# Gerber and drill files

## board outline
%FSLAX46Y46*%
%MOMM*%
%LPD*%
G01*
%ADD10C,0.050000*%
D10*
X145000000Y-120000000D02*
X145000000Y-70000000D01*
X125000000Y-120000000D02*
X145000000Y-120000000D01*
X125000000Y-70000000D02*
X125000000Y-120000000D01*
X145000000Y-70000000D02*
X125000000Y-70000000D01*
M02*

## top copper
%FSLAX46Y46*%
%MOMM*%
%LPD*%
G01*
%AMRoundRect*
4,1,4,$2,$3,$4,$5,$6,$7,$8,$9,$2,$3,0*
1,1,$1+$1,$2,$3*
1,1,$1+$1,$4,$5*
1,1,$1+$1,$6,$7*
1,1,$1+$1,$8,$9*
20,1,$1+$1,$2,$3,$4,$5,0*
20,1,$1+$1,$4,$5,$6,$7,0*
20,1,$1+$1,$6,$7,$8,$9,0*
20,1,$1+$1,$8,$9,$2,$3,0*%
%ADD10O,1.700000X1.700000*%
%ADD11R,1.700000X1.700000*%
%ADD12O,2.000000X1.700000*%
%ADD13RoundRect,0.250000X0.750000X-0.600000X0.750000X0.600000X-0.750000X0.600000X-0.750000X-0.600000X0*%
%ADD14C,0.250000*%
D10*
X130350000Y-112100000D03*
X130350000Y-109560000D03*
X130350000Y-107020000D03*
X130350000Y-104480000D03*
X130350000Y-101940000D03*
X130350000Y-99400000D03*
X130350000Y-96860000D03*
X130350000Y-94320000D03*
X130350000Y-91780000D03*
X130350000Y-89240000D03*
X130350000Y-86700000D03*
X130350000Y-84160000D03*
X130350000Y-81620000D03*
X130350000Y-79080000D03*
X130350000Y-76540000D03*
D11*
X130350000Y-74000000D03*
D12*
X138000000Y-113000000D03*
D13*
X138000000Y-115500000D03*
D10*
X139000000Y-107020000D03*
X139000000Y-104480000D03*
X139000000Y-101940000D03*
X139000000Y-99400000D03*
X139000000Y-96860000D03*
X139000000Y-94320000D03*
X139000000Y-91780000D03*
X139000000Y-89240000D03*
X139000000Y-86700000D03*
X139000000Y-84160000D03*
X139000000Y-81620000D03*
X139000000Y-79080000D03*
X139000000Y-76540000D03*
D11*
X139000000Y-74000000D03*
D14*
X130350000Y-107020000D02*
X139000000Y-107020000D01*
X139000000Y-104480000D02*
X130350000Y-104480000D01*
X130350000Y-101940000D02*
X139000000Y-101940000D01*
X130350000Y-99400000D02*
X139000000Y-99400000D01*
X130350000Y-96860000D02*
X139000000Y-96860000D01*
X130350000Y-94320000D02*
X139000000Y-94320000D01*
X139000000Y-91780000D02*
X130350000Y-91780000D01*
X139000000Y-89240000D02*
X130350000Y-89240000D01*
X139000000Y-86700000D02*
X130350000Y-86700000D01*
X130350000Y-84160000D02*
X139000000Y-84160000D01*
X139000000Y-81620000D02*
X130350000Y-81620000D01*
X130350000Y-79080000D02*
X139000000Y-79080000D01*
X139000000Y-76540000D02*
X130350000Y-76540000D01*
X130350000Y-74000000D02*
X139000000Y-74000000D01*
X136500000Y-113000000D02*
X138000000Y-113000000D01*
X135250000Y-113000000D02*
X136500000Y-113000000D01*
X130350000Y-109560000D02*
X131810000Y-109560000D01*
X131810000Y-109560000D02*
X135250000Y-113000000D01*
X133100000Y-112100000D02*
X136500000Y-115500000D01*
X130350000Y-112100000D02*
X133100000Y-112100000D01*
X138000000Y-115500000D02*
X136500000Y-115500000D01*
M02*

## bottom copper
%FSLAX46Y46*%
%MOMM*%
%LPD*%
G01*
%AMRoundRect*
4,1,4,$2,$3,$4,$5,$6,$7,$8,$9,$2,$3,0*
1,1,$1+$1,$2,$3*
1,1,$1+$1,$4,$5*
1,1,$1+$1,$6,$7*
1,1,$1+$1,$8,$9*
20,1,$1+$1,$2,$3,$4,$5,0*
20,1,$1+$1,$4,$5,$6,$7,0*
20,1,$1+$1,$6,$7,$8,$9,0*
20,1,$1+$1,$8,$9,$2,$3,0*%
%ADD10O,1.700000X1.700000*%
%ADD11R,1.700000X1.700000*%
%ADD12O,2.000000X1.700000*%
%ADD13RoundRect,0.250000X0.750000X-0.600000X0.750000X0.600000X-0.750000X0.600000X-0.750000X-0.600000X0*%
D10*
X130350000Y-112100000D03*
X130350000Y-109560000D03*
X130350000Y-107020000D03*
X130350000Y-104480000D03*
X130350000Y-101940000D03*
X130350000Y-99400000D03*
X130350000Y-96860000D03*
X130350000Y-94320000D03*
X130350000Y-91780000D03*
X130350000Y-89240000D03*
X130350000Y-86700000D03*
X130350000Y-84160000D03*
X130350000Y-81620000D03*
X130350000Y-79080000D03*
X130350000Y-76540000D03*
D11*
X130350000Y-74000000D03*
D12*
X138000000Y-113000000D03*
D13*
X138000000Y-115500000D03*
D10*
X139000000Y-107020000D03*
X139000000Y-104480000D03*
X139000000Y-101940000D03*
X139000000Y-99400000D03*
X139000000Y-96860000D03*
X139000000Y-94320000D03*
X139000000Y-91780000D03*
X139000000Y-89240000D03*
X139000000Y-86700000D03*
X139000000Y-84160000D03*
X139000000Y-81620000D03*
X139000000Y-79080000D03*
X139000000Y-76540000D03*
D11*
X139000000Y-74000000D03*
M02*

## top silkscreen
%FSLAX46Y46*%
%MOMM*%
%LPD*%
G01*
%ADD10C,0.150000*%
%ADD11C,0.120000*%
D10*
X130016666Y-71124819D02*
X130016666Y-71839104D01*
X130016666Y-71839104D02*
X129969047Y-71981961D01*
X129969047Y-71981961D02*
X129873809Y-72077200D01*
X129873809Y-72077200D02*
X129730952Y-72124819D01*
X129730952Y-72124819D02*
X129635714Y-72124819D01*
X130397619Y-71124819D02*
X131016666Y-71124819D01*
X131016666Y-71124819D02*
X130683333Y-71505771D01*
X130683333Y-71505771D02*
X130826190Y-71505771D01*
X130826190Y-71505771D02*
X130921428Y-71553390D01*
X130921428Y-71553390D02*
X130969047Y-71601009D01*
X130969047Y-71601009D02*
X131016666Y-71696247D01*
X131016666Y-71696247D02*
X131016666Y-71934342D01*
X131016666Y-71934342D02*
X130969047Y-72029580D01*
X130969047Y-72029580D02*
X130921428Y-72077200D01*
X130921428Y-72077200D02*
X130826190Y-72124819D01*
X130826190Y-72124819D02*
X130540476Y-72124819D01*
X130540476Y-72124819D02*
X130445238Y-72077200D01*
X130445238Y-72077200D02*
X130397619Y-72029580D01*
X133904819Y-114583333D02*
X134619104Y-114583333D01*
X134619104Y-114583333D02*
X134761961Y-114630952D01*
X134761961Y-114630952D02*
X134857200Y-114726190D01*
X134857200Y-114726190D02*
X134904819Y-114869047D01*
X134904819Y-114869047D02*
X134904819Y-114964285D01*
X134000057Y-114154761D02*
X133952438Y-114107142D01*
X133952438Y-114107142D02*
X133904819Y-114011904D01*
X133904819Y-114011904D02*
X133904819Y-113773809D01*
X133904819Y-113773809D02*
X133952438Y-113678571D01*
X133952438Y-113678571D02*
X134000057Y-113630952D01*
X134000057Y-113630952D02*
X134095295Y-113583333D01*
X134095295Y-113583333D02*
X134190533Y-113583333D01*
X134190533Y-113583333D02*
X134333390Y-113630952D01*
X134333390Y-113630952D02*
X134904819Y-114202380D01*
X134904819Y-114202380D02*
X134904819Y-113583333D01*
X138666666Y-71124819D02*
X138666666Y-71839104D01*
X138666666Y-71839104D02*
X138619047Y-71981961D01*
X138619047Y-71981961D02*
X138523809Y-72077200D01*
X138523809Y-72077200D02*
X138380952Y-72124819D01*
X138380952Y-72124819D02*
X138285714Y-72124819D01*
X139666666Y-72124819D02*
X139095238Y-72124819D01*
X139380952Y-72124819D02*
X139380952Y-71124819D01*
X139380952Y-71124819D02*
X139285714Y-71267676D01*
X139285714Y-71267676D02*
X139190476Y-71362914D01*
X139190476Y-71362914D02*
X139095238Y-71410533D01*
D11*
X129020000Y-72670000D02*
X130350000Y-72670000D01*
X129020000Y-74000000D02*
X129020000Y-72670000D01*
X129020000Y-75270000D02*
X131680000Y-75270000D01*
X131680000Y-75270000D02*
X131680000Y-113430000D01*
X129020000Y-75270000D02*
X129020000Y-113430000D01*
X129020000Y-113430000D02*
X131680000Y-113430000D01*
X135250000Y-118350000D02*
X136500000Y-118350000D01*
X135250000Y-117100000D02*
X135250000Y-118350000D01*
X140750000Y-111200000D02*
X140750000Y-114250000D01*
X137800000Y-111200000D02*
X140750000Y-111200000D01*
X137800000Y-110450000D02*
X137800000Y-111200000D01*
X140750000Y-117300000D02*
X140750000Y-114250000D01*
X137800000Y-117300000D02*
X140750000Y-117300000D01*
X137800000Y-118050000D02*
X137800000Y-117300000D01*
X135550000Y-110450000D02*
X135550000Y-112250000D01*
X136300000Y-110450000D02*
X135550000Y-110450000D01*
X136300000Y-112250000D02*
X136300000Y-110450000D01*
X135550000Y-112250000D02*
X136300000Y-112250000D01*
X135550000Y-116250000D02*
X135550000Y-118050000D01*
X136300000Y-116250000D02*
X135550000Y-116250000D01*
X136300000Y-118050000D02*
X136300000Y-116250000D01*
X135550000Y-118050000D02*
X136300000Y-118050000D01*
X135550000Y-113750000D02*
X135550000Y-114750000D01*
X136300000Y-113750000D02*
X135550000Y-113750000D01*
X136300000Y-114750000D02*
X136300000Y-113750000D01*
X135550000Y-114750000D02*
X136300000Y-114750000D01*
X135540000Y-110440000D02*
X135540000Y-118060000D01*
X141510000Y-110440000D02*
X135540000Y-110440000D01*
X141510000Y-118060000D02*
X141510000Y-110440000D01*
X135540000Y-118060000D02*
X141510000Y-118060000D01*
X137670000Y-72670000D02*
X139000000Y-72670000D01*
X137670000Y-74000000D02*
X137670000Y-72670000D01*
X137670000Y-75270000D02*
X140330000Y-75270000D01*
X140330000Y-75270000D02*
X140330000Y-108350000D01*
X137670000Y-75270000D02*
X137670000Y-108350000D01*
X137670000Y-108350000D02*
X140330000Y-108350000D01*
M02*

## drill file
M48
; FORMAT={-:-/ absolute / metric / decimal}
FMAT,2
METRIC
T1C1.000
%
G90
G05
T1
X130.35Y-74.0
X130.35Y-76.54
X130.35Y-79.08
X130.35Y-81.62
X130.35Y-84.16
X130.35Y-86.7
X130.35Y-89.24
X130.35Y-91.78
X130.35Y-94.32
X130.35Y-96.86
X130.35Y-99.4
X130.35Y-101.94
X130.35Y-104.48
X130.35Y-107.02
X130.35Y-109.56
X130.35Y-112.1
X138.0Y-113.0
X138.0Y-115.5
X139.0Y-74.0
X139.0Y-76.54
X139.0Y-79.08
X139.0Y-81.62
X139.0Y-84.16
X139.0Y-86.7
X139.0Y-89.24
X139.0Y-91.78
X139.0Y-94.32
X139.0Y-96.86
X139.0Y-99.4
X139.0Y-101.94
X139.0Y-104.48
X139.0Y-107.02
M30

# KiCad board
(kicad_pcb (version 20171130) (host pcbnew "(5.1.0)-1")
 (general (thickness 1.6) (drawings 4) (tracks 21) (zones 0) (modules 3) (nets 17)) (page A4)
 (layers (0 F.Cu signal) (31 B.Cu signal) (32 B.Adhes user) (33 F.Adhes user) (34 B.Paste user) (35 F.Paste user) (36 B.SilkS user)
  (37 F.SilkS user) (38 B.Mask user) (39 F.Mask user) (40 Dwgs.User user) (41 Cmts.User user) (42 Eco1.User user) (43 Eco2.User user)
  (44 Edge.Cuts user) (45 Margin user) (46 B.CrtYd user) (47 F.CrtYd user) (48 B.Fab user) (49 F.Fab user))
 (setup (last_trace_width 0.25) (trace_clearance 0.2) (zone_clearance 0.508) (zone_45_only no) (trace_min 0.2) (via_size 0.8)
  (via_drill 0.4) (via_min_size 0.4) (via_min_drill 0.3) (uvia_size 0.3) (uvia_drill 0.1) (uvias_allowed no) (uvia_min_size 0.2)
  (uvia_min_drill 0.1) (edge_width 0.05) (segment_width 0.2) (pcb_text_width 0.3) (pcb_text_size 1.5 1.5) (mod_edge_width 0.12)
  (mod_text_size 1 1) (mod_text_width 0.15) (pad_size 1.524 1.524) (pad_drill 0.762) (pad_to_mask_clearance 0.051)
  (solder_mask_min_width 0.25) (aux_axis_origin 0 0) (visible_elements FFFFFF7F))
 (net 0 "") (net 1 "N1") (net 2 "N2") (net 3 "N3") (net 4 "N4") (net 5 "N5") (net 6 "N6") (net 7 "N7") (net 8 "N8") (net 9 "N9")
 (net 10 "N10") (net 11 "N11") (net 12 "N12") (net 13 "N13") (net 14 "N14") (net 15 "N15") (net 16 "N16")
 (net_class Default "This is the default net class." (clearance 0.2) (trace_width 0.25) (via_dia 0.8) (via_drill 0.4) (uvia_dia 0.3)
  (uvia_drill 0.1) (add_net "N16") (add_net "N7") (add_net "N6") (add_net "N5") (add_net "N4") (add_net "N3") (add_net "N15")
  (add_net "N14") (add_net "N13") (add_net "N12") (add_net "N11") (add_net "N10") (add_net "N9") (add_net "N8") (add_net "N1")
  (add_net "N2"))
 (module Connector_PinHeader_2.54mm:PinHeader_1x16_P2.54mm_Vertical (layer F.Cu) (at 130.35 74)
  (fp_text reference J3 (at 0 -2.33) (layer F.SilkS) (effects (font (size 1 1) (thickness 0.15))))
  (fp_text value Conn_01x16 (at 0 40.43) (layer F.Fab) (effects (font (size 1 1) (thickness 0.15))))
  (fp_line (start -1.33 -1.33) (end 0 -1.33) (layer F.SilkS) (width 0.12))
  (fp_line (start -1.33 0) (end -1.33 -1.33) (layer F.SilkS) (width 0.12))
  (fp_line (start -1.33 1.27) (end 1.33 1.27) (layer F.SilkS) (width 0.12))
  (fp_line (start 1.33 1.27) (end 1.33 39.43) (layer F.SilkS) (width 0.12))
  (fp_line (start -1.33 1.27) (end -1.33 39.43) (layer F.SilkS) (width 0.12))
  (fp_line (start -1.33 39.43) (end 1.33 39.43) (layer F.SilkS) (width 0.12))
  (pad 16 thru_hole oval (at 0 38.1) (size 1.7 1.7) (drill 1) (layers *.Cu *.Mask) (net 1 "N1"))
  (pad 15 thru_hole oval (at 0 35.56) (size 1.7 1.7) (drill 1) (layers *.Cu *.Mask) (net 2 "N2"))
  (pad 14 thru_hole oval (at 0 33.02) (size 1.7 1.7) (drill 1) (layers *.Cu *.Mask) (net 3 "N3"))
  (pad 13 thru_hole oval (at 0 30.48) (size 1.7 1.7) (drill 1) (layers *.Cu *.Mask) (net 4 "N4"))
  (pad 12 thru_hole oval (at 0 27.94) (size 1.7 1.7) (drill 1) (layers *.Cu *.Mask) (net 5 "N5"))
  (pad 11 thru_hole oval (at 0 25.4) (size 1.7 1.7) (drill 1) (layers *.Cu *.Mask) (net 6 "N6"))
  (pad 10 thru_hole oval (at 0 22.86) (size 1.7 1.7) (drill 1) (layers *.Cu *.Mask) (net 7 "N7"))
  (pad 9 thru_hole oval (at 0 20.32) (size 1.7 1.7) (drill 1) (layers *.Cu *.Mask) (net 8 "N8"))
  (pad 8 thru_hole oval (at 0 17.78) (size 1.7 1.7) (drill 1) (layers *.Cu *.Mask) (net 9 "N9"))
  (pad 7 thru_hole oval (at 0 15.24) (size 1.7 1.7) (drill 1) (layers *.Cu *.Mask) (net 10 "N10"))
  (pad 6 thru_hole oval (at 0 12.7) (size 1.7 1.7) (drill 1) (layers *.Cu *.Mask) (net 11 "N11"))
  (pad 5 thru_hole oval (at 0 10.16) (size 1.7 1.7) (drill 1) (layers *.Cu *.Mask) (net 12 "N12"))
  (pad 4 thru_hole oval (at 0 7.62) (size 1.7 1.7) (drill 1) (layers *.Cu *.Mask) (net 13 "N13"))
  (pad 3 thru_hole oval (at 0 5.08) (size 1.7 1.7) (drill 1) (layers *.Cu *.Mask) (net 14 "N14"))
  (pad 2 thru_hole oval (at 0 2.54) (size 1.7 1.7) (drill 1) (layers *.Cu *.Mask) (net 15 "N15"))
  (pad 1 thru_hole rect (at 0 0) (size 1.7 1.7) (drill 1) (layers *.Cu *.Mask) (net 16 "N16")))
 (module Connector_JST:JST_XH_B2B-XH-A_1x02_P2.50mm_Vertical (layer F.Cu) (at 138 115.5 90)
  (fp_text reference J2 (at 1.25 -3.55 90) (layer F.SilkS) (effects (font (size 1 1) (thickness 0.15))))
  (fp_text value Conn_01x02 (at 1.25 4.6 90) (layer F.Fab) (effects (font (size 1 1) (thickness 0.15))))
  (fp_line (start -2.85 -2.75) (end -2.85 -1.5) (layer F.SilkS) (width 0.12))
  (fp_line (start -1.6 -2.75) (end -2.85 -2.75) (layer F.SilkS) (width 0.12))
  (fp_line (start 4.3 2.75) (end 1.25 2.75) (layer F.SilkS) (width 0.12))
  (fp_line (start 4.3 -0.2) (end 4.3 2.75) (layer F.SilkS) (width 0.12))
  (fp_line (start 5.05 -0.2) (end 4.3 -0.2) (layer F.SilkS) (width 0.12))
  (fp_line (start -1.8 2.75) (end 1.25 2.75) (layer F.SilkS) (width 0.12))
  (fp_line (start -1.8 -0.2) (end -1.8 2.75) (layer F.SilkS) (width 0.12))
  (fp_line (start -2.55 -0.2) (end -1.8 -0.2) (layer F.SilkS) (width 0.12))
  (fp_line (start 5.05 -2.45) (end 3.25 -2.45) (layer F.SilkS) (width 0.12))
  (fp_line (start 5.05 -1.7) (end 5.05 -2.45) (layer F.SilkS) (width 0.12))
  (fp_line (start 3.25 -1.7) (end 5.05 -1.7) (layer F.SilkS) (width 0.12))
  (fp_line (start 3.25 -2.45) (end 3.25 -1.7) (layer F.SilkS) (width 0.12))
  (fp_line (start -0.75 -2.45) (end -2.55 -2.45) (layer F.SilkS) (width 0.12))
  (fp_line (start -0.75 -1.7) (end -0.75 -2.45) (layer F.SilkS) (width 0.12))
  (fp_line (start -2.55 -1.7) (end -0.75 -1.7) (layer F.SilkS) (width 0.12))
  (fp_line (start -2.55 -2.45) (end -2.55 -1.7) (layer F.SilkS) (width 0.12))
  (fp_line (start 1.75 -2.45) (end 0.75 -2.45) (layer F.SilkS) (width 0.12))
  (fp_line (start 1.75 -1.7) (end 1.75 -2.45) (layer F.SilkS) (width 0.12))
  (fp_line (start 0.75 -1.7) (end 1.75 -1.7) (layer F.SilkS) (width 0.12))
  (fp_line (start 0.75 -2.45) (end 0.75 -1.7) (layer F.SilkS) (width 0.12))
  (fp_line (start 5.06 -2.46) (end -2.56 -2.46) (layer F.SilkS) (width 0.12))
  (fp_line (start 5.06 3.51) (end 5.06 -2.46) (layer F.SilkS) (width 0.12))
  (fp_line (start -2.56 3.51) (end 5.06 3.51) (layer F.SilkS) (width 0.12))
  (fp_line (start -2.56 -2.46) (end -2.56 3.51) (layer F.SilkS) (width 0.12))
  (pad 2 thru_hole oval (at 2.5 0 90) (size 1.7 2) (drill 1) (layers *.Cu *.Mask) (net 2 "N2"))
  (pad 1 thru_hole roundrect (at 0 0 90) (size 1.7 2) (drill 1) (layers *.Cu *.Mask) (roundrect_rratio 0.147059) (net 1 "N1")))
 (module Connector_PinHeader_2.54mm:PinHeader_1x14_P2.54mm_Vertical (layer F.Cu) (at 139 74)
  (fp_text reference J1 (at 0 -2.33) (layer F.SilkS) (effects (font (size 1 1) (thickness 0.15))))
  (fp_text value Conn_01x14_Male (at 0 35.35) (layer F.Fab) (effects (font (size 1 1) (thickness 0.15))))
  (fp_line (start -1.33 -1.33) (end 0 -1.33) (layer F.SilkS) (width 0.12))
  (fp_line (start -1.33 0) (end -1.33 -1.33) (layer F.SilkS) (width 0.12))
  (fp_line (start -1.33 1.27) (end 1.33 1.27) (layer F.SilkS) (width 0.12))
  (fp_line (start 1.33 1.27) (end 1.33 34.35) (layer F.SilkS) (width 0.12))
  (fp_line (start -1.33 1.27) (end -1.33 34.35) (layer F.SilkS) (width 0.12))
  (fp_line (start -1.33 34.35) (end 1.33 34.35) (layer F.SilkS) (width 0.12))
  (pad 14 thru_hole oval (at 0 33.02) (size 1.7 1.7) (drill 1) (layers *.Cu *.Mask) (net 3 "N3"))
  (pad 13 thru_hole oval (at 0 30.48) (size 1.7 1.7) (drill 1) (layers *.Cu *.Mask) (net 4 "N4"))
  (pad 12 thru_hole oval (at 0 27.94) (size 1.7 1.7) (drill 1) (layers *.Cu *.Mask) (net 5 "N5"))
  (pad 11 thru_hole oval (at 0 25.4) (size 1.7 1.7) (drill 1) (layers *.Cu *.Mask) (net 6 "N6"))
  (pad 10 thru_hole oval (at 0 22.86) (size 1.7 1.7) (drill 1) (layers *.Cu *.Mask) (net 7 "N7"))
  (pad 9 thru_hole oval (at 0 20.32) (size 1.7 1.7) (drill 1) (layers *.Cu *.Mask) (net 8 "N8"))
  (pad 8 thru_hole oval (at 0 17.78) (size 1.7 1.7) (drill 1) (layers *.Cu *.Mask) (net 9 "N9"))
  (pad 7 thru_hole oval (at 0 15.24) (size 1.7 1.7) (drill 1) (layers *.Cu *.Mask) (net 10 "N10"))
  (pad 6 thru_hole oval (at 0 12.7) (size 1.7 1.7) (drill 1) (layers *.Cu *.Mask) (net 11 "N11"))
  (pad 5 thru_hole oval (at 0 10.16) (size 1.7 1.7) (drill 1) (layers *.Cu *.Mask) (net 12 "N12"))
  (pad 4 thru_hole oval (at 0 7.62) (size 1.7 1.7) (drill 1) (layers *.Cu *.Mask) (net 13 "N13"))
  (pad 3 thru_hole oval (at 0 5.08) (size 1.7 1.7) (drill 1) (layers *.Cu *.Mask) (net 14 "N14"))
  (pad 2 thru_hole oval (at 0 2.54) (size 1.7 1.7) (drill 1) (layers *.Cu *.Mask) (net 15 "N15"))
  (pad 1 thru_hole rect (at 0 0) (size 1.7 1.7) (drill 1) (layers *.Cu *.Mask) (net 16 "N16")))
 (gr_line (start 145 120) (end 145 70) (layer Edge.Cuts) (width 0.05))
 (gr_line (start 125 120) (end 145 120) (layer Edge.Cuts) (width 0.05))
 (gr_line (start 125 70) (end 125 120) (layer Edge.Cuts) (width 0.05))
 (gr_line (start 145 70) (end 125 70) (layer Edge.Cuts) (width 0.05))
 (segment (start 130.35 107.02) (end 139 107.02) (width 0.25) (layer F.Cu) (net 3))
 (segment (start 139 104.48) (end 130.35 104.48) (width 0.25) (layer F.Cu) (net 4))
 (segment (start 130.35 101.94) (end 139 101.94) (width 0.25) (layer F.Cu) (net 5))
 (segment (start 130.35 99.4) (end 139 99.4) (width 0.25) (layer F.Cu) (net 6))
 (segment (start 130.35 96.86) (end 139 96.86) (width 0.25) (layer F.Cu) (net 7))
 (segment (start 130.35 94.32) (end 139 94.32) (width 0.25) (layer F.Cu) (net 8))
 (segment (start 139 91.78) (end 130.35 91.78) (width 0.25) (layer F.Cu) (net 9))
 (segment (start 139 89.24) (end 130.35 89.24) (width 0.25) (layer F.Cu) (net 10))
 (segment (start 139 86.7) (end 130.35 86.7) (width 0.25) (layer F.Cu) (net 11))
 (segment (start 130.35 84.16) (end 139 84.16) (width 0.25) (layer F.Cu) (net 12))
 (segment (start 139 81.62) (end 130.35 81.62) (width 0.25) (layer F.Cu) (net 13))
 (segment (start 130.35 79.08) (end 139 79.08) (width 0.25) (layer F.Cu) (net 14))
 (segment (start 139 76.54) (end 130.35 76.54) (width 0.25) (layer F.Cu) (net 15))
 (segment (start 130.35 74) (end 139 74) (width 0.25) (layer F.Cu) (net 16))
 (segment (start 136.5 113) (end 138 113) (width 0.25) (layer F.Cu) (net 2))
 (segment (start 135.25 113) (end 136.5 113) (width 0.25) (layer F.Cu) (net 2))
 (segment (start 130.35 109.56) (end 131.81 109.56) (width 0.25) (layer F.Cu) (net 2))
 (segment (start 131.81 109.56) (end 135.25 113) (width 0.25) (layer F.Cu) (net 2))
 (segment (start 133.1 112.1) (end 136.5 115.5) (width 0.25) (layer F.Cu) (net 1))
 (segment (start 130.35 112.1) (end 133.1 112.1) (width 0.25) (layer F.Cu) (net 1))
 (segment (start 138 115.5) (end 136.5 115.5) (width 0.25) (layer F.Cu) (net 1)))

